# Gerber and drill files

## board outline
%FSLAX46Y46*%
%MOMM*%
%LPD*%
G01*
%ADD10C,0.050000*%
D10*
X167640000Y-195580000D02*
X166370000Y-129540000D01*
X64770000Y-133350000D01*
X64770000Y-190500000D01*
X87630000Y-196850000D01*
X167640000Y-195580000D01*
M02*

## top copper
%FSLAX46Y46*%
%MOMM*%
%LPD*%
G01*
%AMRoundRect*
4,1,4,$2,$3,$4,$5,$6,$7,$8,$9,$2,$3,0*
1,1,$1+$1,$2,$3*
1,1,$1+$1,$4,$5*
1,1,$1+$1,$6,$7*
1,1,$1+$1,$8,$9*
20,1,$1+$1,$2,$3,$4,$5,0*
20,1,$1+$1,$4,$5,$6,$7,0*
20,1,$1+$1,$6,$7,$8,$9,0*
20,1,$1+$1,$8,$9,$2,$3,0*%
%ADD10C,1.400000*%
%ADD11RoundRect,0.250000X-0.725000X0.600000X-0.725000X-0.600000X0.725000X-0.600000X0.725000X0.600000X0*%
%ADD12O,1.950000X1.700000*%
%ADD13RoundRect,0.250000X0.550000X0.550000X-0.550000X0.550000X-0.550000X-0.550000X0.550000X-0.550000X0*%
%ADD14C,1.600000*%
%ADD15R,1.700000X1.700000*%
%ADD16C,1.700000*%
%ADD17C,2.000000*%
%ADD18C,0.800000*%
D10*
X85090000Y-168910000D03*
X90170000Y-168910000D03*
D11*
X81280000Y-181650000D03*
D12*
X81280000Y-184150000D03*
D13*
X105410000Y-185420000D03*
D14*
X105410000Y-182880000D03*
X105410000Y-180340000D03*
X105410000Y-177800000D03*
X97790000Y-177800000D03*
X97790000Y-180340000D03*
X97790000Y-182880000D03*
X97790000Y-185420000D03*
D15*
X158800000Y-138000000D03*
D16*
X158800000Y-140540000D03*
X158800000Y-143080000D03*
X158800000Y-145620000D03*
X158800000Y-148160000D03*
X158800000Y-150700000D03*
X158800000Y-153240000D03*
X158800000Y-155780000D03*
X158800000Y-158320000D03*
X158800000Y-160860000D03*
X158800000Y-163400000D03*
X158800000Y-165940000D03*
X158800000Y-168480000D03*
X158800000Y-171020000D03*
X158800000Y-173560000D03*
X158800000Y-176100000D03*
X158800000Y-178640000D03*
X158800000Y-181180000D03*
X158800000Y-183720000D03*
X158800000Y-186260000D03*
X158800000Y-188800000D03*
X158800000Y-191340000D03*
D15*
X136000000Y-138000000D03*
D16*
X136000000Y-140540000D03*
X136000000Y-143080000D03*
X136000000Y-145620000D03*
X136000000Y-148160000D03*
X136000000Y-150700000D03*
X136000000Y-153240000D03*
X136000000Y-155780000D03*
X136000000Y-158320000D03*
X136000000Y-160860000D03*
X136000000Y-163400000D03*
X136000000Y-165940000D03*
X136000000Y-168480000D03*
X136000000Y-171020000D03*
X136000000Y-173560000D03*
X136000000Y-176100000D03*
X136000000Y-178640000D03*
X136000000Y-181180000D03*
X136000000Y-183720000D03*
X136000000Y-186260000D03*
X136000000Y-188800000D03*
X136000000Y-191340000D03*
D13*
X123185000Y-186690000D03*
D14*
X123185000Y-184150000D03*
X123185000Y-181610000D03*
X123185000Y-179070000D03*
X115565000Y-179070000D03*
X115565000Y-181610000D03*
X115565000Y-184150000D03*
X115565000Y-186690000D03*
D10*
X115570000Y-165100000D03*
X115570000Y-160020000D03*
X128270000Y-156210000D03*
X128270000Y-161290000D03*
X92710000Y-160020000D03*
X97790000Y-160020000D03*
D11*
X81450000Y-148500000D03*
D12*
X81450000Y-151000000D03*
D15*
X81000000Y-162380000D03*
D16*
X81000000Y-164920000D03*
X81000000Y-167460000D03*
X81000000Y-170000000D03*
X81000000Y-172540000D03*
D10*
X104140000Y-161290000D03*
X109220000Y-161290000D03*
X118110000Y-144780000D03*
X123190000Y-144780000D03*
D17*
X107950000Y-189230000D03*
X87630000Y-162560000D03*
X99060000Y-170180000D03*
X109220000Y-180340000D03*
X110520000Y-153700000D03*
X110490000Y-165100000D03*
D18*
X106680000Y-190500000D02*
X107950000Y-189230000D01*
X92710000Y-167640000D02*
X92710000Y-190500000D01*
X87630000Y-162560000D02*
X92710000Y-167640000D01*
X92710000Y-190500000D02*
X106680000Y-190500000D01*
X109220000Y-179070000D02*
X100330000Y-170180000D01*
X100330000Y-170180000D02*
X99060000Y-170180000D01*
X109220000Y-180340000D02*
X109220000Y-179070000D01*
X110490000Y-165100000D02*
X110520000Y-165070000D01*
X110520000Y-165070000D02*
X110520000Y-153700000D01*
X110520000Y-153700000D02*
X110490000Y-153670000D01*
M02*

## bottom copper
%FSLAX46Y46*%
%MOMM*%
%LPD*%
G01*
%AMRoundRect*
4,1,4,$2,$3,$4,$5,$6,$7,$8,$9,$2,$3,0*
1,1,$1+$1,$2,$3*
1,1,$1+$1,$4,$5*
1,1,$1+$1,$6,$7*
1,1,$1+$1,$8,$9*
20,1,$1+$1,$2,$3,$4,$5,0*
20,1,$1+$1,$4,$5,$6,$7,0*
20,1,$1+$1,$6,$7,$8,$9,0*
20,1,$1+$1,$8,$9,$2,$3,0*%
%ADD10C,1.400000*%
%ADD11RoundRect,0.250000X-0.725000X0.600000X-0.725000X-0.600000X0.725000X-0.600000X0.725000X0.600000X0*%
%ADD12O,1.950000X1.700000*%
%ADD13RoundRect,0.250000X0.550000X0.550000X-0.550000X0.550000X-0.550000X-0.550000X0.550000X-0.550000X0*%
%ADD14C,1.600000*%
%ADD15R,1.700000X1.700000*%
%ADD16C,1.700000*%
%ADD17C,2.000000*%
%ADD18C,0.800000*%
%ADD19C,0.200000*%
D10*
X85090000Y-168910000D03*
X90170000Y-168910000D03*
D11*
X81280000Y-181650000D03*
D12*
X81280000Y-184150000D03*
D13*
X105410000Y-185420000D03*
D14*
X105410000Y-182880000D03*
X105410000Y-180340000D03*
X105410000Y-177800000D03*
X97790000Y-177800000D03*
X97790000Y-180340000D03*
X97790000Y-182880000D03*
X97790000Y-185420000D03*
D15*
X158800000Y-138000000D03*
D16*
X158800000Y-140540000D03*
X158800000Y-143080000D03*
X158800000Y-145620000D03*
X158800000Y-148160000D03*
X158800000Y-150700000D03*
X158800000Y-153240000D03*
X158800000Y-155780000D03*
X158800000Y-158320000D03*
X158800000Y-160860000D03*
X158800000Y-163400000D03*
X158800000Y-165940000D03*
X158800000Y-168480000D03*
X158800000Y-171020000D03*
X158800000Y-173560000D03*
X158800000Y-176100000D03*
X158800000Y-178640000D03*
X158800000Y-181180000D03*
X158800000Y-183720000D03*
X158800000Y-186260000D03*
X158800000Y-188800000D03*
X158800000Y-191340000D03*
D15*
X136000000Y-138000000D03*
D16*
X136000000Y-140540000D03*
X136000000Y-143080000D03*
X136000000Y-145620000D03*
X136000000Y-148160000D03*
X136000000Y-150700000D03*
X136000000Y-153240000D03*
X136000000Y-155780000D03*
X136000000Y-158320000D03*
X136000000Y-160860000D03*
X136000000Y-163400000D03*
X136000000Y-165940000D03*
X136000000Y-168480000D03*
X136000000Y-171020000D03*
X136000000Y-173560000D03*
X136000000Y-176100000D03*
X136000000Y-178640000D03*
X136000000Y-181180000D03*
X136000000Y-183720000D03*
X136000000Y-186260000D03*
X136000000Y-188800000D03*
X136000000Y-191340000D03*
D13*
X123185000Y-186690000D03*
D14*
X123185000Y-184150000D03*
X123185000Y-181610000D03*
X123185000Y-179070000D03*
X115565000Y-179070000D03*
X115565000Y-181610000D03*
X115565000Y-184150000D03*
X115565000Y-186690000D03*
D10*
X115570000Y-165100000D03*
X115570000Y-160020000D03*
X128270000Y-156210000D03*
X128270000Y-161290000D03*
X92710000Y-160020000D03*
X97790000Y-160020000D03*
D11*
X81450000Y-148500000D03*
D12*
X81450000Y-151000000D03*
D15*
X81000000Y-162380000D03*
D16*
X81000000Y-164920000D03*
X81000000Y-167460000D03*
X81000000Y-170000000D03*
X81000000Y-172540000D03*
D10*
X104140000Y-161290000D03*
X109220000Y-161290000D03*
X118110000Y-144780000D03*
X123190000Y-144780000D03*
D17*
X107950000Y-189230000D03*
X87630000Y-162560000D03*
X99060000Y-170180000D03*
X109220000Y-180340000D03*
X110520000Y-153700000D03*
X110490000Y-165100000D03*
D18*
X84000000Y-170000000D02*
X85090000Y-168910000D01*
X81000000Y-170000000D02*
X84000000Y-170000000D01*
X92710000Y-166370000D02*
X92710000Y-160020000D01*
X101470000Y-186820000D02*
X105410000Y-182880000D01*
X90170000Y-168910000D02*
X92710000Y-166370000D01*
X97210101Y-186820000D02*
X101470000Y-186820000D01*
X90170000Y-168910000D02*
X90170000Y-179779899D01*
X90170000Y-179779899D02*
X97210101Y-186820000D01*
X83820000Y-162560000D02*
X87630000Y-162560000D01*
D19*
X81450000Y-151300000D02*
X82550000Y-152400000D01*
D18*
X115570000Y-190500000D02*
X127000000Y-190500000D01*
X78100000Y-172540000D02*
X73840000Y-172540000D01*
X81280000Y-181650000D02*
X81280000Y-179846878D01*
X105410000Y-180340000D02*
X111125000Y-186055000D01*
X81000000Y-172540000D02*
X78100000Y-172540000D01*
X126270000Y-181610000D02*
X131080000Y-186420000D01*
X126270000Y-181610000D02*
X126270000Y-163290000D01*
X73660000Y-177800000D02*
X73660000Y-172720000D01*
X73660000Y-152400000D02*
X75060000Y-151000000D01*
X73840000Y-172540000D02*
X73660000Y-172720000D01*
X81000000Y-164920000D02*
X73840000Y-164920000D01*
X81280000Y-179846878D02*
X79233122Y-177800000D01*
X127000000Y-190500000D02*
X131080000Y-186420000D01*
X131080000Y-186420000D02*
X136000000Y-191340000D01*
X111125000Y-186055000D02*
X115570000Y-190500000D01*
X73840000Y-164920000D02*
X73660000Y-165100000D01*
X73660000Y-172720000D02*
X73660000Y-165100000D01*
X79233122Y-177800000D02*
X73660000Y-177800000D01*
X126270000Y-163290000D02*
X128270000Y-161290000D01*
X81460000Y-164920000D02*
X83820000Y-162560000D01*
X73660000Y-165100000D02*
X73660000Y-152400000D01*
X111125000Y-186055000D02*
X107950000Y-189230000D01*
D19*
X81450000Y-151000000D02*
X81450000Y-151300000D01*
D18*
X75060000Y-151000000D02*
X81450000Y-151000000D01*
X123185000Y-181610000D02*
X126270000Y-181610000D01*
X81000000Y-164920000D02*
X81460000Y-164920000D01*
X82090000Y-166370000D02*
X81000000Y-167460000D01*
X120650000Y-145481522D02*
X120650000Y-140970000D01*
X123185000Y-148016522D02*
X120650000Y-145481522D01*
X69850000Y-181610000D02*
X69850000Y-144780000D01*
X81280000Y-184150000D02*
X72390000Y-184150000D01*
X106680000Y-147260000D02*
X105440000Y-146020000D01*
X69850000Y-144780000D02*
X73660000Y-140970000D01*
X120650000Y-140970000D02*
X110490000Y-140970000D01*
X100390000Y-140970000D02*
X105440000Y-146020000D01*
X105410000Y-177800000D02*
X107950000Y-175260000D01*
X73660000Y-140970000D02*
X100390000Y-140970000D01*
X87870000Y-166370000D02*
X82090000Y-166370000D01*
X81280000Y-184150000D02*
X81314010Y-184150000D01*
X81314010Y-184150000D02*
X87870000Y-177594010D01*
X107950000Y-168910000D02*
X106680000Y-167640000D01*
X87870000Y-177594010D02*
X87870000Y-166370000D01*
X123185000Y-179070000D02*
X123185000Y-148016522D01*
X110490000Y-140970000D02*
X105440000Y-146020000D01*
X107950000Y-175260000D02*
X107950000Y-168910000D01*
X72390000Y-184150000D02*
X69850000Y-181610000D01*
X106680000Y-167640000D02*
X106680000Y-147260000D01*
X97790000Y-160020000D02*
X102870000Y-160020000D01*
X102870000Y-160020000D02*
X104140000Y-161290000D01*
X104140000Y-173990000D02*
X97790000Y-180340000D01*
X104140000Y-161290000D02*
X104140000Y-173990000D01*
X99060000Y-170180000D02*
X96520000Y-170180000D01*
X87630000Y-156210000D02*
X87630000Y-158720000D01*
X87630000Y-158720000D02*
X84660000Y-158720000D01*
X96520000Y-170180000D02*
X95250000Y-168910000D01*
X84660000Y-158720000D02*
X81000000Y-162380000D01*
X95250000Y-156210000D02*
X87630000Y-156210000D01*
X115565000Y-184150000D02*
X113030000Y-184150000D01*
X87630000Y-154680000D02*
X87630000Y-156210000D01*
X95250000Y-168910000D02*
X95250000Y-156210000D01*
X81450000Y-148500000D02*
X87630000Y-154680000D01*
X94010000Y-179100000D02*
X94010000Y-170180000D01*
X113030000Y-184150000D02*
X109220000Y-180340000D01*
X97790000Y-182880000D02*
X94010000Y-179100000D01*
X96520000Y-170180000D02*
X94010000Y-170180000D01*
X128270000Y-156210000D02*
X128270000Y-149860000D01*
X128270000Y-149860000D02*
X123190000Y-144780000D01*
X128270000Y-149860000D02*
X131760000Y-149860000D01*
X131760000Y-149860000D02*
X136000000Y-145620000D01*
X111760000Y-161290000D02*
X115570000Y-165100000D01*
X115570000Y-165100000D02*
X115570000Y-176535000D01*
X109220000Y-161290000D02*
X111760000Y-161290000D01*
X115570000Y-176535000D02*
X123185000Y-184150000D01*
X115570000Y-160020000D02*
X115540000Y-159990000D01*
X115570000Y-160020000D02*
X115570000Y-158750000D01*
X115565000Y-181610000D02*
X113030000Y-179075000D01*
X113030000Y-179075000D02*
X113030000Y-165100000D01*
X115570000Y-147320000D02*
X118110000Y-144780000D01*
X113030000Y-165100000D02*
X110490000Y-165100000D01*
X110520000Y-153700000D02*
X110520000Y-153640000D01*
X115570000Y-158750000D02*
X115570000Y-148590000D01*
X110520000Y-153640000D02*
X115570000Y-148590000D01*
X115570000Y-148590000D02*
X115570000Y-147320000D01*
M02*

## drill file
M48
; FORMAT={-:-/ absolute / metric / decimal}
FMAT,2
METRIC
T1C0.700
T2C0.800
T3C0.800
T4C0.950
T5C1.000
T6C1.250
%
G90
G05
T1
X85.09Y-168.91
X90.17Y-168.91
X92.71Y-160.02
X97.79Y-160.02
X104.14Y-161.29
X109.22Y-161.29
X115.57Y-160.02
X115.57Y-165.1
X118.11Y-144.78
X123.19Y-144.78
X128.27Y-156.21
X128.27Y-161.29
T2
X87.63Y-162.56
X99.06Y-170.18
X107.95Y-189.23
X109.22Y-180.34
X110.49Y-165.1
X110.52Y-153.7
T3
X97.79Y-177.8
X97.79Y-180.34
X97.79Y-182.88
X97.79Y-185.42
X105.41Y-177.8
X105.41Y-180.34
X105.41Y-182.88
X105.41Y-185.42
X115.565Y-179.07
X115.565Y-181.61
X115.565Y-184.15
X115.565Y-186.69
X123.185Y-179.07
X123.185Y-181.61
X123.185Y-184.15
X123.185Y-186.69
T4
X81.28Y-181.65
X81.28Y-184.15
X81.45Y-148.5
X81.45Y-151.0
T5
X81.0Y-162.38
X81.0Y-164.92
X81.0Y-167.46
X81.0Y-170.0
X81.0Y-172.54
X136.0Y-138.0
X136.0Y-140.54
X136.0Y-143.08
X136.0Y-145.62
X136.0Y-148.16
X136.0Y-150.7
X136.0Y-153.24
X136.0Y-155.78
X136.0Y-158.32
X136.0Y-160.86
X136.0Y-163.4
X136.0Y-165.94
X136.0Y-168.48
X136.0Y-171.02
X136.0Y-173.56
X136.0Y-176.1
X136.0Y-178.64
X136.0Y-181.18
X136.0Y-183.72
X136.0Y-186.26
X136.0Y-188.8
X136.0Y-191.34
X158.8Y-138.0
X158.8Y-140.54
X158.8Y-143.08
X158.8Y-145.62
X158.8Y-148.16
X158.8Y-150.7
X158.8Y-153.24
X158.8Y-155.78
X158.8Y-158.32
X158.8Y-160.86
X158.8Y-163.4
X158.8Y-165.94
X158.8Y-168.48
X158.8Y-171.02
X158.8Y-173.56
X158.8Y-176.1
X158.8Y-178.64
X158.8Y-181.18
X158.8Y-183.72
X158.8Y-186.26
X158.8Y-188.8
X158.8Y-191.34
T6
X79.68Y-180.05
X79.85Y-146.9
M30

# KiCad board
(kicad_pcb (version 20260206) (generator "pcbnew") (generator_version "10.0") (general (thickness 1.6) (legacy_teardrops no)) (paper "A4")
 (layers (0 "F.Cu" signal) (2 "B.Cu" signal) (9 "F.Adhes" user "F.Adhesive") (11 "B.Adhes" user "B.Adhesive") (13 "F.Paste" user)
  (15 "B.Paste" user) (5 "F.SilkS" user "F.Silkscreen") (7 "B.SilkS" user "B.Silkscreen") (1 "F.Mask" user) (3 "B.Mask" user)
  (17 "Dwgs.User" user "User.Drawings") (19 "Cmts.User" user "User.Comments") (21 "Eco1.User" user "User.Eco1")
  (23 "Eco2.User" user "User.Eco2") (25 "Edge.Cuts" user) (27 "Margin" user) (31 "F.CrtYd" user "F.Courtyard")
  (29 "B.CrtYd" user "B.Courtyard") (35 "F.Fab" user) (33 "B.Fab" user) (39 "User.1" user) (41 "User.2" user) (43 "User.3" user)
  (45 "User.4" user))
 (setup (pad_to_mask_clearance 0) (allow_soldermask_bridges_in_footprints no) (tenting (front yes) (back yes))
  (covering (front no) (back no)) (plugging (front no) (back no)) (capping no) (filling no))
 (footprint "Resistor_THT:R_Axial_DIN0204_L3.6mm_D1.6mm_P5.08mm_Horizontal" (layer "F.Cu") (at 85.09 168.91)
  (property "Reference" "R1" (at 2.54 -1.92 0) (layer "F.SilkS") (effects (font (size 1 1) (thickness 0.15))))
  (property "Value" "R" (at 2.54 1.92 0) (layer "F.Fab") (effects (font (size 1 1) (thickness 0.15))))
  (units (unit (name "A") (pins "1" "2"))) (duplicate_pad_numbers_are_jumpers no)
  (pad "1" thru_hole circle (at 0 0) (size 1.4 1.4) (drill 0.7) (layers "*.Cu" "*.Mask") (remove_unused_layers no) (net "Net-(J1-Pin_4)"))
  (pad "2" thru_hole circle (at 5.08 0) (size 1.4 1.4) (drill 0.7) (layers "*.Cu" "*.Mask") (remove_unused_layers no) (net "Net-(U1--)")))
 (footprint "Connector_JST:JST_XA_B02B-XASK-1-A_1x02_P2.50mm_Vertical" (layer "F.Cu") (at 81.28 181.65 -90)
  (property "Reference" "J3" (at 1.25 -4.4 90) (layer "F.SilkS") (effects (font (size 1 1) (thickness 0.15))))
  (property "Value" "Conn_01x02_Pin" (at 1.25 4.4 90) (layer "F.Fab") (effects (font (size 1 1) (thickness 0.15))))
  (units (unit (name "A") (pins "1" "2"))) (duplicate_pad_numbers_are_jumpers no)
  (pad "" np_thru_hole circle (at -1.6 1.6 270) (size 1.25 1.25) (drill 1.25) (layers "*.Cu" "*.Mask"))
  (pad "1" thru_hole roundrect (at 0 0 270) (size 1.7 1.95) (drill 0.95) (layers "*.Cu" "*.Mask") (remove_unused_layers no)
   (roundrect_rratio 0.147059) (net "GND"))
  (pad "2" thru_hole oval (at 2.5 0 270) (size 1.7 1.95) (drill 0.95) (layers "*.Cu" "*.Mask") (remove_unused_layers no) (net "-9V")))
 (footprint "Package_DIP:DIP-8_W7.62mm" (layer "F.Cu") (at 105.41 185.42 180)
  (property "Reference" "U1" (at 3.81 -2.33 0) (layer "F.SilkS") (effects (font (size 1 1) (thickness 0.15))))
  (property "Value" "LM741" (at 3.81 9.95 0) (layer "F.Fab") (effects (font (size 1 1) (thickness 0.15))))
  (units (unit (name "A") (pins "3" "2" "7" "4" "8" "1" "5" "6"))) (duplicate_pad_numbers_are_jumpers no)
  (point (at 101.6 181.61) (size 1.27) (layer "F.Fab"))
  (pad "1" thru_hole roundrect (at 0 0 180) (size 1.6 1.6) (drill 0.8) (layers "*.Cu" "*.Mask") (remove_unused_layers no)
   (roundrect_rratio 0.15625) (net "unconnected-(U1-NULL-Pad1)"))
  (pad "2" thru_hole circle (at 0 2.54 180) (size 1.6 1.6) (drill 0.8) (layers "*.Cu" "*.Mask") (remove_unused_layers no) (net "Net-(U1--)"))
  (pad "3" thru_hole circle (at 0 5.08 180) (size 1.6 1.6) (drill 0.8) (layers "*.Cu" "*.Mask") (remove_unused_layers no) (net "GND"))
  (pad "4" thru_hole circle (at 0 7.62 180) (size 1.6 1.6) (drill 0.8) (layers "*.Cu" "*.Mask") (remove_unused_layers no) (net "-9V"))
  (pad "5" thru_hole circle (at 7.62 7.62 180) (size 1.6 1.6) (drill 0.8) (layers "*.Cu" "*.Mask") (remove_unused_layers no)
   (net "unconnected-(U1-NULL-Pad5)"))
  (pad "6" thru_hole circle (at 7.62 5.08 180) (size 1.6 1.6) (drill 0.8) (layers "*.Cu" "*.Mask") (remove_unused_layers no)
   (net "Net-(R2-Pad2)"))
  (pad "7" thru_hole circle (at 7.62 2.54 180) (size 1.6 1.6) (drill 0.8) (layers "*.Cu" "*.Mask") (remove_unused_layers no) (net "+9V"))
  (pad "8" thru_hole circle (at 7.62 0 180) (size 1.6 1.6) (drill 0.8) (layers "*.Cu" "*.Mask") (remove_unused_layers no)
   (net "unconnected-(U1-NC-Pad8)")))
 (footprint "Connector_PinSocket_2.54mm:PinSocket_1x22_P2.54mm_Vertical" (layer "F.Cu") (at 158.8 138)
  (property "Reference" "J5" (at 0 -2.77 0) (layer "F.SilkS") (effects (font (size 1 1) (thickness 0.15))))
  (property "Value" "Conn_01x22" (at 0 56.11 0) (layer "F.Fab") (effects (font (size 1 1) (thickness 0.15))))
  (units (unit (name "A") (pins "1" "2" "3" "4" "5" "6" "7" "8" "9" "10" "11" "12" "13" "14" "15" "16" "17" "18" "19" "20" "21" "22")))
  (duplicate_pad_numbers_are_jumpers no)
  (pad "1" thru_hole rect (at 0 0) (size 1.7 1.7) (drill 1) (layers "*.Cu" "*.Mask") (remove_unused_layers no)
   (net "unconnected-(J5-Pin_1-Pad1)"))
  (pad "2" thru_hole circle (at 0 2.54) (size 1.7 1.7) (drill 1) (layers "*.Cu" "*.Mask") (remove_unused_layers no)
   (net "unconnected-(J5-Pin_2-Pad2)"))
  (pad "3" thru_hole circle (at 0 5.08) (size 1.7 1.7) (drill 1) (layers "*.Cu" "*.Mask") (remove_unused_layers no)
   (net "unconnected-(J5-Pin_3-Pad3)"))
  (pad "4" thru_hole circle (at 0 7.62) (size 1.7 1.7) (drill 1) (layers "*.Cu" "*.Mask") (remove_unused_layers no)
   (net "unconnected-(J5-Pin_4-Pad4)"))
  (pad "5" thru_hole circle (at 0 10.16) (size 1.7 1.7) (drill 1) (layers "*.Cu" "*.Mask") (remove_unused_layers no)
   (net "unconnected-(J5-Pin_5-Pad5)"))
  (pad "6" thru_hole circle (at 0 12.7) (size 1.7 1.7) (drill 1) (layers "*.Cu" "*.Mask") (remove_unused_layers no)
   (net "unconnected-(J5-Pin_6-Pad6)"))
  (pad "7" thru_hole circle (at 0 15.24) (size 1.7 1.7) (drill 1) (layers "*.Cu" "*.Mask") (remove_unused_layers no)
   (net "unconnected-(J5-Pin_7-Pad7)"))
  (pad "8" thru_hole circle (at 0 17.78) (size 1.7 1.7) (drill 1) (layers "*.Cu" "*.Mask") (remove_unused_layers no)
   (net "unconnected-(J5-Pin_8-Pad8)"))
  (pad "9" thru_hole circle (at 0 20.32) (size 1.7 1.7) (drill 1) (layers "*.Cu" "*.Mask") (remove_unused_layers no)
   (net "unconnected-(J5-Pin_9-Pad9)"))
  (pad "10" thru_hole circle (at 0 22.86) (size 1.7 1.7) (drill 1) (layers "*.Cu" "*.Mask") (remove_unused_layers no)
   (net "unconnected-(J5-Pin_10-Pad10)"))
  (pad "11" thru_hole circle (at 0 25.4) (size 1.7 1.7) (drill 1) (layers "*.Cu" "*.Mask") (remove_unused_layers no)
   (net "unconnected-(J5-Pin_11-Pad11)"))
  (pad "12" thru_hole circle (at 0 27.94) (size 1.7 1.7) (drill 1) (layers "*.Cu" "*.Mask") (remove_unused_layers no)
   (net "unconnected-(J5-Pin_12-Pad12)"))
  (pad "13" thru_hole circle (at 0 30.48) (size 1.7 1.7) (drill 1) (layers "*.Cu" "*.Mask") (remove_unused_layers no)
   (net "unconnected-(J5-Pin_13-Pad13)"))
  (pad "14" thru_hole circle (at 0 33.02) (size 1.7 1.7) (drill 1) (layers "*.Cu" "*.Mask") (remove_unused_layers no)
   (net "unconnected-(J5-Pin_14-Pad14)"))
  (pad "15" thru_hole circle (at 0 35.56) (size 1.7 1.7) (drill 1) (layers "*.Cu" "*.Mask") (remove_unused_layers no)
   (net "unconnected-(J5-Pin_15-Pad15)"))
  (pad "16" thru_hole circle (at 0 38.1) (size 1.7 1.7) (drill 1) (layers "*.Cu" "*.Mask") (remove_unused_layers no)
   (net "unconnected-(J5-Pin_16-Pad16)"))
  (pad "17" thru_hole circle (at 0 40.64) (size 1.7 1.7) (drill 1) (layers "*.Cu" "*.Mask") (remove_unused_layers no)
   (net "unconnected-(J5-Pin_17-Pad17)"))
  (pad "18" thru_hole circle (at 0 43.18) (size 1.7 1.7) (drill 1) (layers "*.Cu" "*.Mask") (remove_unused_layers no)
   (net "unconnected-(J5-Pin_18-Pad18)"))
  (pad "19" thru_hole circle (at 0 45.72) (size 1.7 1.7) (drill 1) (layers "*.Cu" "*.Mask") (remove_unused_layers no)
   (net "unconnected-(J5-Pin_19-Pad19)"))
  (pad "20" thru_hole circle (at 0 48.26) (size 1.7 1.7) (drill 1) (layers "*.Cu" "*.Mask") (remove_unused_layers no)
   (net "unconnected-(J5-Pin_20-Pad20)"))
  (pad "21" thru_hole circle (at 0 50.8) (size 1.7 1.7) (drill 1) (layers "*.Cu" "*.Mask") (remove_unused_layers no)
   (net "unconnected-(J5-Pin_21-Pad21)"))
  (pad "22" thru_hole circle (at 0 53.34) (size 1.7 1.7) (drill 1) (layers "*.Cu" "*.Mask") (remove_unused_layers no)
   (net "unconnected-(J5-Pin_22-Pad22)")))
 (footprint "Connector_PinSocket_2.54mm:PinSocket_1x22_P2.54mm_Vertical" (layer "F.Cu") (at 136 138)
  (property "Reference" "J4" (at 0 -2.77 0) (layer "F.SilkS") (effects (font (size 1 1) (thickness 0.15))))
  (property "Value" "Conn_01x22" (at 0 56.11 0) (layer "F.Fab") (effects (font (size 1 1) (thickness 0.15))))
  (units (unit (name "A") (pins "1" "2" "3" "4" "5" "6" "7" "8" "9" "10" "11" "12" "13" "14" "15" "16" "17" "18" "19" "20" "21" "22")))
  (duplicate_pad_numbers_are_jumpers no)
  (pad "1" thru_hole rect (at 0 0) (size 1.7 1.7) (drill 1) (layers "*.Cu" "*.Mask") (remove_unused_layers no)
   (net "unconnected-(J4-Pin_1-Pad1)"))
  (pad "2" thru_hole circle (at 0 2.54) (size 1.7 1.7) (drill 1) (layers "*.Cu" "*.Mask") (remove_unused_layers no)
   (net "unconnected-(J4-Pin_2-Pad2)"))
  (pad "3" thru_hole circle (at 0 5.08) (size 1.7 1.7) (drill 1) (layers "*.Cu" "*.Mask") (remove_unused_layers no)
   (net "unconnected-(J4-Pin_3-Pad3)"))
  (pad "4" thru_hole circle (at 0 7.62) (size 1.7 1.7) (drill 1) (layers "*.Cu" "*.Mask") (remove_unused_layers no) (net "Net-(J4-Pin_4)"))
  (pad "5" thru_hole circle (at 0 10.16) (size 1.7 1.7) (drill 1) (layers "*.Cu" "*.Mask") (remove_unused_layers no)
   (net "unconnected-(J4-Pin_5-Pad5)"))
  (pad "6" thru_hole circle (at 0 12.7) (size 1.7 1.7) (drill 1) (layers "*.Cu" "*.Mask") (remove_unused_layers no)
   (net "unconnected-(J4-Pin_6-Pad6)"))
  (pad "7" thru_hole circle (at 0 15.24) (size 1.7 1.7) (drill 1) (layers "*.Cu" "*.Mask") (remove_unused_layers no)
   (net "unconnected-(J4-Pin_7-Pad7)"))
  (pad "8" thru_hole circle (at 0 17.78) (size 1.7 1.7) (drill 1) (layers "*.Cu" "*.Mask") (remove_unused_layers no)
   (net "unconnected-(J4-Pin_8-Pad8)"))
  (pad "9" thru_hole circle (at 0 20.32) (size 1.7 1.7) (drill 1) (layers "*.Cu" "*.Mask") (remove_unused_layers no)
   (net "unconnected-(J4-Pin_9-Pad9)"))
  (pad "10" thru_hole circle (at 0 22.86) (size 1.7 1.7) (drill 1) (layers "*.Cu" "*.Mask") (remove_unused_layers no)
   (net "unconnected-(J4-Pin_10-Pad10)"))
  (pad "11" thru_hole circle (at 0 25.4) (size 1.7 1.7) (drill 1) (layers "*.Cu" "*.Mask") (remove_unused_layers no)
   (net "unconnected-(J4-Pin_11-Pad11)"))
  (pad "12" thru_hole circle (at 0 27.94) (size 1.7 1.7) (drill 1) (layers "*.Cu" "*.Mask") (remove_unused_layers no)
   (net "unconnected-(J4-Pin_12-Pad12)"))
  (pad "13" thru_hole circle (at 0 30.48) (size 1.7 1.7) (drill 1) (layers "*.Cu" "*.Mask") (remove_unused_layers no)
   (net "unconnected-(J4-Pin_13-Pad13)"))
  (pad "14" thru_hole circle (at 0 33.02) (size 1.7 1.7) (drill 1) (layers "*.Cu" "*.Mask") (remove_unused_layers no)
   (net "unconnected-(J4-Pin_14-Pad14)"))
  (pad "15" thru_hole circle (at 0 35.56) (size 1.7 1.7) (drill 1) (layers "*.Cu" "*.Mask") (remove_unused_layers no)
   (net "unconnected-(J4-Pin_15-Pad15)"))
  (pad "16" thru_hole circle (at 0 38.1) (size 1.7 1.7) (drill 1) (layers "*.Cu" "*.Mask") (remove_unused_layers no)
   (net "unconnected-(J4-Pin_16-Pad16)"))
  (pad "17" thru_hole circle (at 0 40.64) (size 1.7 1.7) (drill 1) (layers "*.Cu" "*.Mask") (remove_unused_layers no)
   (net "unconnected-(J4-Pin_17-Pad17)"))
  (pad "18" thru_hole circle (at 0 43.18) (size 1.7 1.7) (drill 1) (layers "*.Cu" "*.Mask") (remove_unused_layers no)
   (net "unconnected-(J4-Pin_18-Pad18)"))
  (pad "19" thru_hole circle (at 0 45.72) (size 1.7 1.7) (drill 1) (layers "*.Cu" "*.Mask") (remove_unused_layers no)
   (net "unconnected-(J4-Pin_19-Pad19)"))
  (pad "20" thru_hole circle (at 0 48.26) (size 1.7 1.7) (drill 1) (layers "*.Cu" "*.Mask") (remove_unused_layers no)
   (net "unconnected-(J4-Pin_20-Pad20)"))
  (pad "21" thru_hole circle (at 0 50.8) (size 1.7 1.7) (drill 1) (layers "*.Cu" "*.Mask") (remove_unused_layers no)
   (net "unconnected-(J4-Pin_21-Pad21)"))
  (pad "22" thru_hole circle (at 0 53.34) (size 1.7 1.7) (drill 1) (layers "*.Cu" "*.Mask") (remove_unused_layers no) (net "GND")))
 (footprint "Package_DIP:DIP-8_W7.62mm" (layer "F.Cu") (at 123.185 186.69 180)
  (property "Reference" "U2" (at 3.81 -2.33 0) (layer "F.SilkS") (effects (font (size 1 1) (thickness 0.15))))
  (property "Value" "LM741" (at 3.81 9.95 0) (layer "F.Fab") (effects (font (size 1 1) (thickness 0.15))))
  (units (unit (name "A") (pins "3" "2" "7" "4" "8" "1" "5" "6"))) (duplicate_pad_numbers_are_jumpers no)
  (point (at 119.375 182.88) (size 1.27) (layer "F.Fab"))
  (pad "1" thru_hole roundrect (at 0 0 180) (size 1.6 1.6) (drill 0.8) (layers "*.Cu" "*.Mask") (remove_unused_layers no)
   (roundrect_rratio 0.15625) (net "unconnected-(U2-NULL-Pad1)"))
  (pad "2" thru_hole circle (at 0 2.54 180) (size 1.6 1.6) (drill 0.8) (layers "*.Cu" "*.Mask") (remove_unused_layers no) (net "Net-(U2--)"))
  (pad "3" thru_hole circle (at 0 5.08 180) (size 1.6 1.6) (drill 0.8) (layers "*.Cu" "*.Mask") (remove_unused_layers no) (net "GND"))
  (pad "4" thru_hole circle (at 0 7.62 180) (size 1.6 1.6) (drill 0.8) (layers "*.Cu" "*.Mask") (remove_unused_layers no) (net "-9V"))
  (pad "5" thru_hole circle (at 7.62 7.62 180) (size 1.6 1.6) (drill 0.8) (layers "*.Cu" "*.Mask") (remove_unused_layers no)
   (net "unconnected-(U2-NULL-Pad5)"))
  (pad "6" thru_hole circle (at 7.62 5.08 180) (size 1.6 1.6) (drill 0.8) (layers "*.Cu" "*.Mask") (remove_unused_layers no)
   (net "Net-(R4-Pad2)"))
  (pad "7" thru_hole circle (at 7.62 2.54 180) (size 1.6 1.6) (drill 0.8) (layers "*.Cu" "*.Mask") (remove_unused_layers no) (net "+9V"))
  (pad "8" thru_hole circle (at 7.62 0 180) (size 1.6 1.6) (drill 0.8) (layers "*.Cu" "*.Mask") (remove_unused_layers no)
   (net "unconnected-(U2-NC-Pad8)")))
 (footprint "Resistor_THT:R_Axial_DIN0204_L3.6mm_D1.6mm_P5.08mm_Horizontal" (layer "F.Cu") (at 115.57 165.1 90)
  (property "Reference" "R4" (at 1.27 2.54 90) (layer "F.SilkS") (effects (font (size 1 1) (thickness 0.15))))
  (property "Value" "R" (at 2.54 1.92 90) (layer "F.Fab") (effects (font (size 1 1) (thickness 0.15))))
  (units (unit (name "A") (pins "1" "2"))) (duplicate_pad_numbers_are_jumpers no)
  (pad "1" thru_hole circle (at 0 0 90) (size 1.4 1.4) (drill 0.7) (layers "*.Cu" "*.Mask") (remove_unused_layers no) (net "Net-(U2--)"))
  (pad "2" thru_hole circle (at 5.08 0 90) (size 1.4 1.4) (drill 0.7) (layers "*.Cu" "*.Mask") (remove_unused_layers no)
   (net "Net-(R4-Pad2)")))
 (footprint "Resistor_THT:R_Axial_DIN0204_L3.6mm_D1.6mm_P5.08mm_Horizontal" (layer "F.Cu") (at 128.27 156.21 -90)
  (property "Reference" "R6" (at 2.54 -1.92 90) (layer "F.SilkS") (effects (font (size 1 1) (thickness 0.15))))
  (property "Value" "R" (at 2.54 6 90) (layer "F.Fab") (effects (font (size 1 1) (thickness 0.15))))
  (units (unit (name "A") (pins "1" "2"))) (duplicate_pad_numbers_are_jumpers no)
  (pad "1" thru_hole circle (at 0 0 270) (size 1.4 1.4) (drill 0.7) (layers "*.Cu" "*.Mask") (remove_unused_layers no)
   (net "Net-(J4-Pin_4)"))
  (pad "2" thru_hole circle (at 5.08 0 270) (size 1.4 1.4) (drill 0.7) (layers "*.Cu" "*.Mask") (remove_unused_layers no) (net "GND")))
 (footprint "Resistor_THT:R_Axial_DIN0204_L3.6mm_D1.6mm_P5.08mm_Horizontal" (layer "F.Cu") (at 92.71 160.02)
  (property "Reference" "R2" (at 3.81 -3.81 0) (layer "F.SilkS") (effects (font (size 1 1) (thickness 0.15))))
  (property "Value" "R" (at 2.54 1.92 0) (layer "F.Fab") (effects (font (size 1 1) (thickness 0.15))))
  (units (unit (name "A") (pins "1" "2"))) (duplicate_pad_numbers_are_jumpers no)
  (pad "1" thru_hole circle (at 0 0) (size 1.4 1.4) (drill 0.7) (layers "*.Cu" "*.Mask") (remove_unused_layers no) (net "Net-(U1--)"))
  (pad "2" thru_hole circle (at 5.08 0) (size 1.4 1.4) (drill 0.7) (layers "*.Cu" "*.Mask") (remove_unused_layers no) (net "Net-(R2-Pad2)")))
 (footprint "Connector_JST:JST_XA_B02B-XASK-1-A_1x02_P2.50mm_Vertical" (layer "F.Cu") (at 81.45 148.5 -90)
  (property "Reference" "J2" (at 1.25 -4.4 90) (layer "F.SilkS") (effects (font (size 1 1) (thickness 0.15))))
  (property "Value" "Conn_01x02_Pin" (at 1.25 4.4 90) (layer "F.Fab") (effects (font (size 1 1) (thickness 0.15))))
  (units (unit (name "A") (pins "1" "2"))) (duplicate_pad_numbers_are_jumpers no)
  (pad "" np_thru_hole circle (at -1.6 1.6 270) (size 1.25 1.25) (drill 1.25) (layers "*.Cu" "*.Mask"))
  (pad "1" thru_hole roundrect (at 0 0 270) (size 1.7 1.95) (drill 0.95) (layers "*.Cu" "*.Mask") (remove_unused_layers no)
   (roundrect_rratio 0.147059) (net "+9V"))
  (pad "2" thru_hole oval (at 2.5 0 270) (size 1.7 1.95) (drill 0.95) (layers "*.Cu" "*.Mask") (remove_unused_layers no) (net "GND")))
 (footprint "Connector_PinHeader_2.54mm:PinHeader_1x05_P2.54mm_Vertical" (layer "F.Cu") (at 81 162.38)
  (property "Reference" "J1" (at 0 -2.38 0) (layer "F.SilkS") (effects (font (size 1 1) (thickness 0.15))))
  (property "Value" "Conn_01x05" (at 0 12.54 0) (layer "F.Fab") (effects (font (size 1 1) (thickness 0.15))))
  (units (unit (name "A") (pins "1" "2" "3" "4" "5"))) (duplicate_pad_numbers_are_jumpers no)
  (pad "1" thru_hole rect (at 0 0) (size 1.7 1.7) (drill 1) (layers "*.Cu" "*.Mask") (remove_unused_layers no) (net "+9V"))
  (pad "2" thru_hole circle (at 0 2.54) (size 1.7 1.7) (drill 1) (layers "*.Cu" "*.Mask") (remove_unused_layers no) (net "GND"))
  (pad "3" thru_hole circle (at 0 5.08) (size 1.7 1.7) (drill 1) (layers "*.Cu" "*.Mask") (remove_unused_layers no) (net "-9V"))
  (pad "4" thru_hole circle (at 0 7.62) (size 1.7 1.7) (drill 1) (layers "*.Cu" "*.Mask") (remove_unused_layers no) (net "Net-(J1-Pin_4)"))
  (pad "5" thru_hole circle (at 0 10.16) (size 1.7 1.7) (drill 1) (layers "*.Cu" "*.Mask") (remove_unused_layers no) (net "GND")))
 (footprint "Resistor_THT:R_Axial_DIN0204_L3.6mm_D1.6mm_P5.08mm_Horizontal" (layer "F.Cu") (at 104.14 161.29)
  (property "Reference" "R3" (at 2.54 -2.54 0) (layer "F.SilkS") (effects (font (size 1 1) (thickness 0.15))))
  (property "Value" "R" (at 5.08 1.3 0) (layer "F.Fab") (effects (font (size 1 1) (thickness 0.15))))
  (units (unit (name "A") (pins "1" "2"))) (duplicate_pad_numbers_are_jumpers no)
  (pad "1" thru_hole circle (at 0 0) (size 1.4 1.4) (drill 0.7) (layers "*.Cu" "*.Mask") (remove_unused_layers no) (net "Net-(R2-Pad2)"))
  (pad "2" thru_hole circle (at 5.08 0) (size 1.4 1.4) (drill 0.7) (layers "*.Cu" "*.Mask") (remove_unused_layers no) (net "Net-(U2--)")))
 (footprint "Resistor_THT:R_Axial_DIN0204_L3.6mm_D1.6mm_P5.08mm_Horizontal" (layer "F.Cu") (at 118.11 144.78)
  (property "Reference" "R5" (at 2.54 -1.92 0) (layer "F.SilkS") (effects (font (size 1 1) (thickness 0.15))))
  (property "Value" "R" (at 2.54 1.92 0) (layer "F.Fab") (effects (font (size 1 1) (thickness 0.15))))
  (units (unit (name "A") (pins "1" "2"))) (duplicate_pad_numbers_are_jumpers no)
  (pad "1" thru_hole circle (at 0 0) (size 1.4 1.4) (drill 0.7) (layers "*.Cu" "*.Mask") (remove_unused_layers no) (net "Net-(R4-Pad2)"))
  (pad "2" thru_hole circle (at 5.08 0) (size 1.4 1.4) (drill 0.7) (layers "*.Cu" "*.Mask") (remove_unused_layers no) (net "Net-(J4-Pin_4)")))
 (gr_poly
  (pts (xy 167.64 195.58) (xy 166.37 129.54) (xy 64.77 133.35) (xy 64.77 190.5) (xy 87.63 196.85)) (stroke (width 0.05) (type solid))
  (fill no) (layer "Edge.Cuts"))
 (segment (start 84 170) (end 85.09 168.91) (width 0.8) (layer "B.Cu") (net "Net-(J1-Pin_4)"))
 (segment (start 81 170) (end 84 170) (width 0.8) (layer "B.Cu") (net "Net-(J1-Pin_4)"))
 (segment (start 92.71 166.37) (end 92.71 160.02) (width 0.8) (layer "B.Cu") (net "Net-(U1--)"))
 (segment (start 101.47 186.82) (end 105.41 182.88) (width 0.8) (layer "B.Cu") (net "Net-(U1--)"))
 (segment (start 90.17 168.91) (end 92.71 166.37) (width 0.8) (layer "B.Cu") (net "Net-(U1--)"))
 (segment (start 97.210101 186.82) (end 101.47 186.82) (width 0.8) (layer "B.Cu") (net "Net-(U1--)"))
 (segment (start 90.17 168.91) (end 90.17 179.779899) (width 0.8) (layer "B.Cu") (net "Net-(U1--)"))
 (segment (start 90.17 179.779899) (end 97.210101 186.82) (width 0.8) (layer "B.Cu") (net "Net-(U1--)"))
 (segment (start 106.68 190.5) (end 107.95 189.23) (width 0.8) (layer "F.Cu") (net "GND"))
 (segment (start 92.71 167.64) (end 92.71 190.5) (width 0.8) (layer "F.Cu") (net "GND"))
 (segment (start 87.63 162.56) (end 92.71 167.64) (width 0.8) (layer "F.Cu") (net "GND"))
 (segment (start 92.71 190.5) (end 106.68 190.5) (width 0.8) (layer "F.Cu") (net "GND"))
 (via (at 107.95 189.23) (size 2) (drill 0.8) (layers "F.Cu" "B.Cu") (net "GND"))
 (via (at 87.63 162.56) (size 2) (drill 0.8) (layers "F.Cu" "B.Cu") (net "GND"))
 (segment (start 83.82 162.56) (end 87.63 162.56) (width 0.8) (layer "B.Cu") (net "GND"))
 (segment (start 81.45 151.3) (end 82.55 152.4) (width 0.2) (layer "B.Cu") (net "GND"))
 (segment (start 115.57 190.5) (end 127 190.5) (width 0.8) (layer "B.Cu") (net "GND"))
 (segment (start 78.1 172.54) (end 73.84 172.54) (width 0.8) (layer "B.Cu") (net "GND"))
 (segment (start 81.28 181.65) (end 81.28 179.846878) (width 0.8) (layer "B.Cu") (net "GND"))
 (segment (start 105.41 180.34) (end 111.125 186.055) (width 0.8) (layer "B.Cu") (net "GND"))
 (segment (start 81 172.54) (end 78.1 172.54) (width 0.8) (layer "B.Cu") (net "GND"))
 (segment (start 126.27 181.61) (end 131.08 186.42) (width 0.8) (layer "B.Cu") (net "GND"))
 (segment (start 126.27 181.61) (end 126.27 163.29) (width 0.8) (layer "B.Cu") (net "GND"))
 (segment (start 73.66 177.8) (end 73.66 172.72) (width 0.8) (layer "B.Cu") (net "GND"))
 (segment (start 73.66 152.4) (end 75.06 151) (width 0.8) (layer "B.Cu") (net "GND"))
 (segment (start 73.84 172.54) (end 73.66 172.72) (width 0.8) (layer "B.Cu") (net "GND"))
 (segment (start 81 164.92) (end 73.84 164.92) (width 0.8) (layer "B.Cu") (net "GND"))
 (segment (start 81.28 179.846878) (end 79.233122 177.8) (width 0.8) (layer "B.Cu") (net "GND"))
 (segment (start 127 190.5) (end 131.08 186.42) (width 0.8) (layer "B.Cu") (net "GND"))
 (segment (start 131.08 186.42) (end 136 191.34) (width 0.8) (layer "B.Cu") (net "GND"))
 (segment (start 111.125 186.055) (end 115.57 190.5) (width 0.8) (layer "B.Cu") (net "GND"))
 (segment (start 73.84 164.92) (end 73.66 165.1) (width 0.8) (layer "B.Cu") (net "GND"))
 (segment (start 73.66 172.72) (end 73.66 165.1) (width 0.8) (layer "B.Cu") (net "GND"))
 (segment (start 79.233122 177.8) (end 73.66 177.8) (width 0.8) (layer "B.Cu") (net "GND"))
 (segment (start 126.27 163.29) (end 128.27 161.29) (width 0.8) (layer "B.Cu") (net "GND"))
 (segment (start 81.46 164.92) (end 83.82 162.56) (width 0.8) (layer "B.Cu") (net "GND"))
 (segment (start 73.66 165.1) (end 73.66 152.4) (width 0.8) (layer "B.Cu") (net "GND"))
 (segment (start 111.125 186.055) (end 107.95 189.23) (width 0.8) (layer "B.Cu") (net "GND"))
 (segment (start 81.45 151) (end 81.45 151.3) (width 0.2) (layer "B.Cu") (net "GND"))
 (segment (start 75.06 151) (end 81.45 151) (width 0.8) (layer "B.Cu") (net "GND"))
 (segment (start 123.185 181.61) (end 126.27 181.61) (width 0.8) (layer "B.Cu") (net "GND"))
 (segment (start 81 164.92) (end 81.46 164.92) (width 0.8) (layer "B.Cu") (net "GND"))
 (segment (start 82.09 166.37) (end 81 167.46) (width 0.8) (layer "B.Cu") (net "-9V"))
 (segment (start 120.65 145.481522) (end 120.65 140.97) (width 0.8) (layer "B.Cu") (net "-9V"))
 (segment (start 123.185 148.016522) (end 120.65 145.481522) (width 0.8) (layer "B.Cu") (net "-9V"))
 (segment (start 69.85 181.61) (end 69.85 144.78) (width 0.8) (layer "B.Cu") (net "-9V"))
 (segment (start 81.28 184.15) (end 72.39 184.15) (width 0.8) (layer "B.Cu") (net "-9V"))
 (segment (start 106.68 147.26) (end 105.44 146.02) (width 0.8) (layer "B.Cu") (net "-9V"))
 (segment (start 69.85 144.78) (end 73.66 140.97) (width 0.8) (layer "B.Cu") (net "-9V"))
 (segment (start 120.65 140.97) (end 110.49 140.97) (width 0.8) (layer "B.Cu") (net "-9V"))
 (segment (start 100.39 140.97) (end 105.44 146.02) (width 0.8) (layer "B.Cu") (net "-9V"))
 (segment (start 105.41 177.8) (end 107.95 175.26) (width 0.8) (layer "B.Cu") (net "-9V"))
 (segment (start 73.66 140.97) (end 100.39 140.97) (width 0.8) (layer "B.Cu") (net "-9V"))
 (segment (start 87.87 166.37) (end 82.09 166.37) (width 0.8) (layer "B.Cu") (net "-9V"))
 (segment (start 81.28 184.15) (end 81.31401 184.15) (width 0.8) (layer "B.Cu") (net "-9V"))
 (segment (start 81.31401 184.15) (end 87.87 177.59401) (width 0.8) (layer "B.Cu") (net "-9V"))
 (segment (start 107.95 168.91) (end 106.68 167.64) (width 0.8) (layer "B.Cu") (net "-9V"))
 (segment (start 87.87 177.59401) (end 87.87 166.37) (width 0.8) (layer "B.Cu") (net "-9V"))
 (segment (start 123.185 179.07) (end 123.185 148.016522) (width 0.8) (layer "B.Cu") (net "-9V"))
 (segment (start 110.49 140.97) (end 105.44 146.02) (width 0.8) (layer "B.Cu") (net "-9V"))
 (segment (start 107.95 175.26) (end 107.95 168.91) (width 0.8) (layer "B.Cu") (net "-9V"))
 (segment (start 72.39 184.15) (end 69.85 181.61) (width 0.8) (layer "B.Cu") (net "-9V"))
 (segment (start 106.68 167.64) (end 106.68 147.26) (width 0.8) (layer "B.Cu") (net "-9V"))
 (segment (start 97.79 160.02) (end 102.87 160.02) (width 0.8) (layer "B.Cu") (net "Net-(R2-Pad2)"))
 (segment (start 102.87 160.02) (end 104.14 161.29) (width 0.8) (layer "B.Cu") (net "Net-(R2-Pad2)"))
 (segment (start 104.14 173.99) (end 97.79 180.34) (width 0.8) (layer "B.Cu") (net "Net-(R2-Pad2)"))
 (segment (start 104.14 161.29) (end 104.14 173.99) (width 0.8) (layer "B.Cu") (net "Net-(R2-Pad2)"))
 (segment (start 109.22 179.07) (end 100.33 170.18) (width 0.8) (layer "F.Cu") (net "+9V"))
 (segment (start 100.33 170.18) (end 99.06 170.18) (width 0.8) (layer "F.Cu") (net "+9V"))
 (segment (start 109.22 180.34) (end 109.22 179.07) (width 0.8) (layer "F.Cu") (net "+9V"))
 (via (at 99.06 170.18) (size 2) (drill 0.8) (layers "F.Cu" "B.Cu") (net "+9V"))
 (via (at 109.22 180.34) (size 2) (drill 0.8) (layers "F.Cu" "B.Cu") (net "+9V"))
 (segment (start 99.06 170.18) (end 96.52 170.18) (width 0.8) (layer "B.Cu") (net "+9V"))
 (segment (start 87.63 156.21) (end 87.63 158.72) (width 0.8) (layer "B.Cu") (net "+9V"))
 (segment (start 87.63 158.72) (end 84.66 158.72) (width 0.8) (layer "B.Cu") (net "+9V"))
 (segment (start 96.52 170.18) (end 95.25 168.91) (width 0.8) (layer "B.Cu") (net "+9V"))
 (segment (start 84.66 158.72) (end 81 162.38) (width 0.8) (layer "B.Cu") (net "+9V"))
 (segment (start 95.25 156.21) (end 87.63 156.21) (width 0.8) (layer "B.Cu") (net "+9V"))
 (segment (start 115.565 184.15) (end 113.03 184.15) (width 0.8) (layer "B.Cu") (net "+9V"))
 (segment (start 87.63 154.68) (end 87.63 156.21) (width 0.8) (layer "B.Cu") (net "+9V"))
 (segment (start 95.25 168.91) (end 95.25 156.21) (width 0.8) (layer "B.Cu") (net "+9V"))
 (segment (start 81.45 148.5) (end 87.63 154.68) (width 0.8) (layer "B.Cu") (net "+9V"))
 (segment (start 94.01 179.1) (end 94.01 170.18) (width 0.8) (layer "B.Cu") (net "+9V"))
 (segment (start 113.03 184.15) (end 109.22 180.34) (width 0.8) (layer "B.Cu") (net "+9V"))
 (segment (start 97.79 182.88) (end 94.01 179.1) (width 0.8) (layer "B.Cu") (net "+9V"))
 (segment (start 96.52 170.18) (end 94.01 170.18) (width 0.8) (layer "B.Cu") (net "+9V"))
 (segment (start 128.27 156.21) (end 128.27 149.86) (width 0.8) (layer "B.Cu") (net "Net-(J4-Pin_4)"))
 (segment (start 128.27 149.86) (end 123.19 144.78) (width 0.8) (layer "B.Cu") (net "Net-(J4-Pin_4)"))
 (segment (start 128.27 149.86) (end 131.76 149.86) (width 0.8) (layer "B.Cu") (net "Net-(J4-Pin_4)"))
 (segment (start 131.76 149.86) (end 136 145.62) (width 0.8) (layer "B.Cu") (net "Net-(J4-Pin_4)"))
 (segment (start 111.76 161.29) (end 115.57 165.1) (width 0.8) (layer "B.Cu") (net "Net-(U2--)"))
 (segment (start 115.57 165.1) (end 115.57 176.535) (width 0.8) (layer "B.Cu") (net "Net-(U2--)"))
 (segment (start 109.22 161.29) (end 111.76 161.29) (width 0.8) (layer "B.Cu") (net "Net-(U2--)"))
 (segment (start 115.57 176.535) (end 123.185 184.15) (width 0.8) (layer "B.Cu") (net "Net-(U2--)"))
 (segment (start 110.49 165.1) (end 110.52 165.07) (width 0.8) (layer "F.Cu") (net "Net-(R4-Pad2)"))
 (segment (start 110.52 165.07) (end 110.52 153.7) (width 0.8) (layer "F.Cu") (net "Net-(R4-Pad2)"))
 (segment (start 110.52 153.7) (end 110.49 153.67) (width 0.8) (layer "F.Cu") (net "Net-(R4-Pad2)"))
 (via (at 110.52 153.7) (size 2) (drill 0.8) (layers "F.Cu" "B.Cu") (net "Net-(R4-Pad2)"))
 (via (at 110.49 165.1) (size 2) (drill 0.8) (layers "F.Cu" "B.Cu") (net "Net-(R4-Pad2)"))
 (segment (start 115.57 160.02) (end 115.54 159.99) (width 0.8) (layer "B.Cu") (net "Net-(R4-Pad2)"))
 (segment (start 115.57 160.02) (end 115.57 158.75) (width 0.8) (layer "B.Cu") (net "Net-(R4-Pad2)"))
 (segment (start 115.565 181.61) (end 113.03 179.075) (width 0.8) (layer "B.Cu") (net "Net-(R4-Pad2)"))
 (segment (start 113.03 179.075) (end 113.03 165.1) (width 0.8) (layer "B.Cu") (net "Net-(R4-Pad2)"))
 (segment (start 115.57 147.32) (end 118.11 144.78) (width 0.8) (layer "B.Cu") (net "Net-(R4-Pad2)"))
 (segment (start 113.03 165.1) (end 110.49 165.1) (width 0.8) (layer "B.Cu") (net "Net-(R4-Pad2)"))
 (segment (start 110.52 153.7) (end 110.52 153.64) (width 0.8) (layer "B.Cu") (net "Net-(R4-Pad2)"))
 (segment (start 115.57 158.75) (end 115.57 148.59) (width 0.8) (layer "B.Cu") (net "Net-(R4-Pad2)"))
 (segment (start 110.52 153.64) (end 115.57 148.59) (width 0.8) (layer "B.Cu") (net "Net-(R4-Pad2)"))
 (segment (start 115.57 148.59) (end 115.57 147.32) (width 0.8) (layer "B.Cu") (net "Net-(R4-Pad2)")))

